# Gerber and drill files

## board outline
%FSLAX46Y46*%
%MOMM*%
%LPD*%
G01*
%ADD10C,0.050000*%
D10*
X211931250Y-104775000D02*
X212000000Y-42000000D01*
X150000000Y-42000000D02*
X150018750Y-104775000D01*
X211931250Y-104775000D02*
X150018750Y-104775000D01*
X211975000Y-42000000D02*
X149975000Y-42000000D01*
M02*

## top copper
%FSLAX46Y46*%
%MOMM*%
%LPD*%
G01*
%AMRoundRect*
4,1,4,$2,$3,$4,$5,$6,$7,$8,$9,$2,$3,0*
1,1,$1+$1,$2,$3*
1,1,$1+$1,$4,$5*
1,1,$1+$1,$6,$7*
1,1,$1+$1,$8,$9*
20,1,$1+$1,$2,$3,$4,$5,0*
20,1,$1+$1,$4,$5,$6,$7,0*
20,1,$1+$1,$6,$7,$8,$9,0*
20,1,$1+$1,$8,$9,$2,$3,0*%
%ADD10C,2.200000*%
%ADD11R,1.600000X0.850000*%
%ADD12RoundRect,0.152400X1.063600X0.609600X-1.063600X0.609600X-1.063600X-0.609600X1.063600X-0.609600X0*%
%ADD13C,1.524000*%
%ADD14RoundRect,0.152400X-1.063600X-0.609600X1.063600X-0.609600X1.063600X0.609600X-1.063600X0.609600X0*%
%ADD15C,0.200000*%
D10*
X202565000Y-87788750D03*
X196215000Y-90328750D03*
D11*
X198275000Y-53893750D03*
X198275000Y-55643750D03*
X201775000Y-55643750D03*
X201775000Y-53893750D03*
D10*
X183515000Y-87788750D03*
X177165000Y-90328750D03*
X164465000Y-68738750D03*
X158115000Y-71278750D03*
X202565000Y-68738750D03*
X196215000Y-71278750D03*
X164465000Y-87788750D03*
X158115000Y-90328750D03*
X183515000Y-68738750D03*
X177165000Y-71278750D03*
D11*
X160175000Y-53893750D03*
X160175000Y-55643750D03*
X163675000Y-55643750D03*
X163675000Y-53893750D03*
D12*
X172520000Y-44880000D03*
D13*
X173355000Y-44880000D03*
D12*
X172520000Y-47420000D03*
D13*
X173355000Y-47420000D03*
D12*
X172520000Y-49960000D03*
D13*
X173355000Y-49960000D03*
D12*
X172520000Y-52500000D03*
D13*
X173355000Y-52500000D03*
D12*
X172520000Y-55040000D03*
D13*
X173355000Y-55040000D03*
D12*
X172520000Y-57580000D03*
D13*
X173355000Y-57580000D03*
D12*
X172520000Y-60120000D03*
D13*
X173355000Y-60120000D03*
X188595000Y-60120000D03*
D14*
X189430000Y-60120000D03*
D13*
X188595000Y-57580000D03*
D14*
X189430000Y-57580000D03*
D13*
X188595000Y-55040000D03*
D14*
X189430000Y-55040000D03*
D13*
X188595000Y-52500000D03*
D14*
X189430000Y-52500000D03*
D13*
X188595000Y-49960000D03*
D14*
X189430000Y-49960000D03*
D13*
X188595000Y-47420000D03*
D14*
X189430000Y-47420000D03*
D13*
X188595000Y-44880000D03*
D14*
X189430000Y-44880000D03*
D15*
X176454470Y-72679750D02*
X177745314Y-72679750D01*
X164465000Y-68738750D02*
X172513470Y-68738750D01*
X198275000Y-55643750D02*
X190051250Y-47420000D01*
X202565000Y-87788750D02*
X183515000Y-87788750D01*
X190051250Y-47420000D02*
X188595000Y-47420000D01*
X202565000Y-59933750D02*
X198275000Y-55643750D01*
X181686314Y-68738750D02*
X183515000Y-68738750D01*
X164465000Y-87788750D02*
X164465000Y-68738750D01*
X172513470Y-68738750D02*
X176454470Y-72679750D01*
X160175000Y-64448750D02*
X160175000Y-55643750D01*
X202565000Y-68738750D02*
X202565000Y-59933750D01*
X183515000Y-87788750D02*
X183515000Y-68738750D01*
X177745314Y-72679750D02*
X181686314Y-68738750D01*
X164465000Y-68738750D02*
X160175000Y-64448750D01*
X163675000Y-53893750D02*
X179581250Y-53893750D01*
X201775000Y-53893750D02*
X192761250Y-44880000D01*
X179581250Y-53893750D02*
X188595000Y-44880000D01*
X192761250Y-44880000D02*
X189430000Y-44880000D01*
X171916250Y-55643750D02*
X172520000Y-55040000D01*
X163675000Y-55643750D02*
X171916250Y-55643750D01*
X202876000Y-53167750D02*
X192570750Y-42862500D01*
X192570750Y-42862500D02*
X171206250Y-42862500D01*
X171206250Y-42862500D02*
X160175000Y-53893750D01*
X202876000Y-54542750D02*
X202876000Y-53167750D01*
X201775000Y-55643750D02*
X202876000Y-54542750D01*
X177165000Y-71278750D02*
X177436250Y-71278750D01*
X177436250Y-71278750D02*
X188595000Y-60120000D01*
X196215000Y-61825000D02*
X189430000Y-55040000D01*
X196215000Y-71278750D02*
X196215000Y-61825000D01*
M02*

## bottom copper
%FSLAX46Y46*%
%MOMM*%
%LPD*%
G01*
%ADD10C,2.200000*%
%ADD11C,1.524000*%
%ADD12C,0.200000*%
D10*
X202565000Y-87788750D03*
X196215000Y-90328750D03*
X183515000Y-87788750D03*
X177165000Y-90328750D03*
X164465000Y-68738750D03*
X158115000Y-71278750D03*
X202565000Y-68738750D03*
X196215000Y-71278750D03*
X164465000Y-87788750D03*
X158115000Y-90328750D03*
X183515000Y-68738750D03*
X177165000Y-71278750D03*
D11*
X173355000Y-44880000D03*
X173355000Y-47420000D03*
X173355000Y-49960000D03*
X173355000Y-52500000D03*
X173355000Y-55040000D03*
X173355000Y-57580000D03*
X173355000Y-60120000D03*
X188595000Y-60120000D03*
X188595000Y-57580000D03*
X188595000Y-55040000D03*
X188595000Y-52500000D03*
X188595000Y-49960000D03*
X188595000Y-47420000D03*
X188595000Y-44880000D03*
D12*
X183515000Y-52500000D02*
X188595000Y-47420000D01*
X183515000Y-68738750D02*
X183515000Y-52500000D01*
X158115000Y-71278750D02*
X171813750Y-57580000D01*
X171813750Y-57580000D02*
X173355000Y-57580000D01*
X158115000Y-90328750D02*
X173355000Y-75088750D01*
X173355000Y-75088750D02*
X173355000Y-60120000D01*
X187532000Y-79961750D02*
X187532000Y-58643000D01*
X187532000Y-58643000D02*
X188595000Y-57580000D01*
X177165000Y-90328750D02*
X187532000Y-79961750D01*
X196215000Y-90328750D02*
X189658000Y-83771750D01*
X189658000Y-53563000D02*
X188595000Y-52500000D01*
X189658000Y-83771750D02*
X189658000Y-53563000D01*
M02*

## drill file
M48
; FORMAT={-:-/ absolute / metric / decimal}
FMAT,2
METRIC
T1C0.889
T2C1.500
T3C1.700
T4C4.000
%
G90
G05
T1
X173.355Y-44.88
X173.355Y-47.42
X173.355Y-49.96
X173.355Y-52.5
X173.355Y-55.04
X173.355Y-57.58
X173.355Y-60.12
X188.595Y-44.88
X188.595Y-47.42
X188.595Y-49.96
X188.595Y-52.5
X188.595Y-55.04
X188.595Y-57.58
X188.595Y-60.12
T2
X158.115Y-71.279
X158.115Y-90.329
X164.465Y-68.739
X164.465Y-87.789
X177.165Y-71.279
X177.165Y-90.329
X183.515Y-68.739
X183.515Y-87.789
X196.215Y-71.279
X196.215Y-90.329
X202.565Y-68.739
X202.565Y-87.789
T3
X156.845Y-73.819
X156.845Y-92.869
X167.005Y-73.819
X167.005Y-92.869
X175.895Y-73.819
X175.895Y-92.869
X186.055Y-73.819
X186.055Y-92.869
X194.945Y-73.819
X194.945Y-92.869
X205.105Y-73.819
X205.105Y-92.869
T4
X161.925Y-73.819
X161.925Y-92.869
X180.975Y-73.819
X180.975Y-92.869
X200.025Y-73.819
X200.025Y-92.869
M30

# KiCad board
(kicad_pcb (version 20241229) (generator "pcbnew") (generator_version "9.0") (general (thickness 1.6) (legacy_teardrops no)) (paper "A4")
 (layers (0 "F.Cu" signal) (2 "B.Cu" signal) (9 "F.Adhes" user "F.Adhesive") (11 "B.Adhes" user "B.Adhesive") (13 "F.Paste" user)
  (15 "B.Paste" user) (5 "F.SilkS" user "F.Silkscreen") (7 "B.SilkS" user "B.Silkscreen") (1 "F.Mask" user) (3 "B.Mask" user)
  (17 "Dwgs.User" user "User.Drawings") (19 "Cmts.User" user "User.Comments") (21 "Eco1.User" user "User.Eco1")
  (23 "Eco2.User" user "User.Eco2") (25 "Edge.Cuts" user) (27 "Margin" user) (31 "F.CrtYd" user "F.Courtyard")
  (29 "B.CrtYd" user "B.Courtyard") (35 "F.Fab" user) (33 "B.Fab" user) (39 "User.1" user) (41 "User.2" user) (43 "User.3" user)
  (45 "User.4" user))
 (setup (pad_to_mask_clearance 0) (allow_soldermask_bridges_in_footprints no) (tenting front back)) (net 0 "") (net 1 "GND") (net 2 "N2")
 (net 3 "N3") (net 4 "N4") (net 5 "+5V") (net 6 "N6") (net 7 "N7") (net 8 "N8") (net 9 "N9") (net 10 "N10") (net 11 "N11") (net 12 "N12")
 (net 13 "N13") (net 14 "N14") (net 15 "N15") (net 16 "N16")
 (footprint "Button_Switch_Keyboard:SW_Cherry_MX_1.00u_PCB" (layer "F.Cu") (at 202.565 87.78875)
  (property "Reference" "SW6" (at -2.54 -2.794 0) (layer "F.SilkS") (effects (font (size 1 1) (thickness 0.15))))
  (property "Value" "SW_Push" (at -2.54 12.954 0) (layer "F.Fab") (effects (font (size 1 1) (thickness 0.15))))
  (pad "" np_thru_hole circle (at -7.62 5.08) (size 1.7 1.7) (drill 1.7) (layers "*.Cu" "*.Mask"))
  (pad "" np_thru_hole circle (at -2.54 5.08) (size 4 4) (drill 4) (layers "*.Cu" "*.Mask"))
  (pad "" np_thru_hole circle (at 2.54 5.08) (size 1.7 1.7) (drill 1.7) (layers "*.Cu" "*.Mask"))
  (pad "1" thru_hole circle (at 0 0) (size 2.2 2.2) (drill 1.5) (layers "*.Cu" "*.Mask") (remove_unused_layers no) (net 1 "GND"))
  (pad "2" thru_hole circle (at -6.35 2.54) (size 2.2 2.2) (drill 1.5) (layers "*.Cu" "*.Mask") (remove_unused_layers no) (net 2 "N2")))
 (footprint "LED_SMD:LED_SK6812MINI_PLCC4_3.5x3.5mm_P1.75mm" (layer "F.Cu") (at 200.025 54.76875)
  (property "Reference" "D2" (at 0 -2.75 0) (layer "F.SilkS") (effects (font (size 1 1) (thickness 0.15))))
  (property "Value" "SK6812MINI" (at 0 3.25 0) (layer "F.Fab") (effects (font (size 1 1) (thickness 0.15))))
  (pad "1" smd rect (at -1.75 -0.875) (size 1.6 0.85) (layers "F.Cu" "F.Mask" "F.Paste") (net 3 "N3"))
  (pad "2" smd rect (at -1.75 0.875) (size 1.6 0.85) (layers "F.Cu" "F.Mask" "F.Paste") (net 1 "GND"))
  (pad "3" smd rect (at 1.75 0.875) (size 1.6 0.85) (layers "F.Cu" "F.Mask" "F.Paste") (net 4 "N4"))
  (pad "4" smd rect (at 1.75 -0.875) (size 1.6 0.85) (layers "F.Cu" "F.Mask" "F.Paste") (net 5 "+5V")))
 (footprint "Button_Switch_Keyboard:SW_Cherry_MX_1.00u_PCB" (layer "F.Cu") (at 183.515 87.78875)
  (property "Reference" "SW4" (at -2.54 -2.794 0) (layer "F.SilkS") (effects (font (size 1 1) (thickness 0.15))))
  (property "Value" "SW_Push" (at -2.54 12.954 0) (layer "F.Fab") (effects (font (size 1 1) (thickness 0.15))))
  (pad "" np_thru_hole circle (at -7.62 5.08) (size 1.7 1.7) (drill 1.7) (layers "*.Cu" "*.Mask"))
  (pad "" np_thru_hole circle (at -2.54 5.08) (size 4 4) (drill 4) (layers "*.Cu" "*.Mask"))
  (pad "" np_thru_hole circle (at 2.54 5.08) (size 1.7 1.7) (drill 1.7) (layers "*.Cu" "*.Mask"))
  (pad "1" thru_hole circle (at 0 0) (size 2.2 2.2) (drill 1.5) (layers "*.Cu" "*.Mask") (remove_unused_layers no) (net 1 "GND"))
  (pad "2" thru_hole circle (at -6.35 2.54) (size 2.2 2.2) (drill 1.5) (layers "*.Cu" "*.Mask") (remove_unused_layers no) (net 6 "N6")))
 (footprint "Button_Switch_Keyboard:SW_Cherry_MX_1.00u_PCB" (layer "F.Cu") (at 164.465 68.73875)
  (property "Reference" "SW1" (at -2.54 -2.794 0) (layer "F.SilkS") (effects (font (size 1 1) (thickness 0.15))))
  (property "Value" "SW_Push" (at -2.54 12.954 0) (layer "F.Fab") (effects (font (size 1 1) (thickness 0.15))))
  (pad "" np_thru_hole circle (at -7.62 5.08) (size 1.7 1.7) (drill 1.7) (layers "*.Cu" "*.Mask"))
  (pad "" np_thru_hole circle (at -2.54 5.08) (size 4 4) (drill 4) (layers "*.Cu" "*.Mask"))
  (pad "" np_thru_hole circle (at 2.54 5.08) (size 1.7 1.7) (drill 1.7) (layers "*.Cu" "*.Mask"))
  (pad "1" thru_hole circle (at 0 0) (size 2.2 2.2) (drill 1.5) (layers "*.Cu" "*.Mask") (remove_unused_layers no) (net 1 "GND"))
  (pad "2" thru_hole circle (at -6.35 2.54) (size 2.2 2.2) (drill 1.5) (layers "*.Cu" "*.Mask") (remove_unused_layers no) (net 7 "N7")))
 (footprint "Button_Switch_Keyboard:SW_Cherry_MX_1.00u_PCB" (layer "F.Cu") (at 202.565 68.73875)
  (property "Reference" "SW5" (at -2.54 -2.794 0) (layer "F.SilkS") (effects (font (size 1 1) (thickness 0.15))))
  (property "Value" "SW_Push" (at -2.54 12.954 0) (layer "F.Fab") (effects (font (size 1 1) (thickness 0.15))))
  (pad "" np_thru_hole circle (at -7.62 5.08) (size 1.7 1.7) (drill 1.7) (layers "*.Cu" "*.Mask"))
  (pad "" np_thru_hole circle (at -2.54 5.08) (size 4 4) (drill 4) (layers "*.Cu" "*.Mask"))
  (pad "" np_thru_hole circle (at 2.54 5.08) (size 1.7 1.7) (drill 1.7) (layers "*.Cu" "*.Mask"))
  (pad "1" thru_hole circle (at 0 0) (size 2.2 2.2) (drill 1.5) (layers "*.Cu" "*.Mask") (remove_unused_layers no) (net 1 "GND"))
  (pad "2" thru_hole circle (at -6.35 2.54) (size 2.2 2.2) (drill 1.5) (layers "*.Cu" "*.Mask") (remove_unused_layers no) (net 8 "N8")))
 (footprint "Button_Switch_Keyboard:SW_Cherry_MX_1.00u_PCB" (layer "F.Cu") (at 164.465 87.78875)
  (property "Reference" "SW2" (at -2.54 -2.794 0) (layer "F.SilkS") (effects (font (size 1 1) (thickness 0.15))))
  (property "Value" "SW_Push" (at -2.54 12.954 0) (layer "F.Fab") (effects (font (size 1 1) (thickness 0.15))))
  (pad "" np_thru_hole circle (at -7.62 5.08) (size 1.7 1.7) (drill 1.7) (layers "*.Cu" "*.Mask"))
  (pad "" np_thru_hole circle (at -2.54 5.08) (size 4 4) (drill 4) (layers "*.Cu" "*.Mask"))
  (pad "" np_thru_hole circle (at 2.54 5.08) (size 1.7 1.7) (drill 1.7) (layers "*.Cu" "*.Mask"))
  (pad "1" thru_hole circle (at 0 0) (size 2.2 2.2) (drill 1.5) (layers "*.Cu" "*.Mask") (remove_unused_layers no) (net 1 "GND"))
  (pad "2" thru_hole circle (at -6.35 2.54) (size 2.2 2.2) (drill 1.5) (layers "*.Cu" "*.Mask") (remove_unused_layers no) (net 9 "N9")))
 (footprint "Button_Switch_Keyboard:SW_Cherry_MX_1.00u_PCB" (layer "F.Cu") (at 183.515 68.73875)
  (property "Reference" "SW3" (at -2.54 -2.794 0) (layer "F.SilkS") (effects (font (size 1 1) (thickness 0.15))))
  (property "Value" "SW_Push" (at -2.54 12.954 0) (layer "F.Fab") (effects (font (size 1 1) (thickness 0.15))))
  (pad "" np_thru_hole circle (at -7.62 5.08) (size 1.7 1.7) (drill 1.7) (layers "*.Cu" "*.Mask"))
  (pad "" np_thru_hole circle (at -2.54 5.08) (size 4 4) (drill 4) (layers "*.Cu" "*.Mask"))
  (pad "" np_thru_hole circle (at 2.54 5.08) (size 1.7 1.7) (drill 1.7) (layers "*.Cu" "*.Mask"))
  (pad "1" thru_hole circle (at 0 0) (size 2.2 2.2) (drill 1.5) (layers "*.Cu" "*.Mask") (remove_unused_layers no) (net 1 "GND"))
  (pad "2" thru_hole circle (at -6.35 2.54) (size 2.2 2.2) (drill 1.5) (layers "*.Cu" "*.Mask") (remove_unused_layers no) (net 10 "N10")))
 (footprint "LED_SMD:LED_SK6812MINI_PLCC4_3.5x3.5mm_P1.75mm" (layer "F.Cu") (at 161.925 54.76875)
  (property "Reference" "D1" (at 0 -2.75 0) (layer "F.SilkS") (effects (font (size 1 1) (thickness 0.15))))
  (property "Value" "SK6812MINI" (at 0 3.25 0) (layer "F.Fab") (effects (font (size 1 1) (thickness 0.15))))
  (pad "1" smd rect (at -1.75 -0.875) (size 1.6 0.85) (layers "F.Cu" "F.Mask" "F.Paste") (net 4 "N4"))
  (pad "2" smd rect (at -1.75 0.875) (size 1.6 0.85) (layers "F.Cu" "F.Mask" "F.Paste") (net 1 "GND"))
  (pad "3" smd rect (at 1.75 0.875) (size 1.6 0.85) (layers "F.Cu" "F.Mask" "F.Paste") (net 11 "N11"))
  (pad "4" smd rect (at 1.75 -0.875) (size 1.6 0.85) (layers "F.Cu" "F.Mask" "F.Paste") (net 5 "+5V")))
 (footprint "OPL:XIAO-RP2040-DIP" (layer "F.Cu") (at 180.975 52.5)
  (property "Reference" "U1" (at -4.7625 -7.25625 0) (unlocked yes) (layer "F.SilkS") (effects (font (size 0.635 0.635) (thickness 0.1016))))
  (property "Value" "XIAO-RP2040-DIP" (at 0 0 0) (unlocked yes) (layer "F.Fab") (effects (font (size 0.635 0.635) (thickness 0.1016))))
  (pad "1" smd roundrect (at -8.455 -7.62 180) (size 2.432 1.524) (layers "F.Cu" "F.Mask") (roundrect_rratio 0.1) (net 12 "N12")
   (thermal_bridge_angle 45))
  (pad "1" thru_hole circle (at -7.62 -7.62 180) (size 1.524 1.524) (drill 0.889) (layers "*.Cu" "*.Mask") (remove_unused_layers no)
   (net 12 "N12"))
  (pad "2" smd roundrect (at -8.455 -5.08 180) (size 2.432 1.524) (layers "F.Cu" "F.Mask") (roundrect_rratio 0.1) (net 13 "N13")
   (thermal_bridge_angle 45))
  (pad "2" thru_hole circle (at -7.62 -5.08 180) (size 1.524 1.524) (drill 0.889) (layers "*.Cu" "*.Mask") (remove_unused_layers no)
   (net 13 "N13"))
  (pad "3" smd roundrect (at -8.455 -2.54 180) (size 2.432 1.524) (layers "F.Cu" "F.Mask") (roundrect_rratio 0.1) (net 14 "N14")
   (thermal_bridge_angle 45))
  (pad "3" thru_hole circle (at -7.62 -2.54 180) (size 1.524 1.524) (drill 0.889) (layers "*.Cu" "*.Mask") (remove_unused_layers no)
   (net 14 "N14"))
  (pad "4" smd roundrect (at -8.455 0 180) (size 2.432 1.524) (layers "F.Cu" "F.Mask") (roundrect_rratio 0.1) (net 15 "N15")
   (thermal_bridge_angle 45))
  (pad "4" thru_hole circle (at -7.62 0 180) (size 1.524 1.524) (drill 0.889) (layers "*.Cu" "*.Mask") (remove_unused_layers no)
   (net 15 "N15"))
  (pad "5" smd roundrect (at -8.455 2.54 180) (size 2.432 1.524) (layers "F.Cu" "F.Mask") (roundrect_rratio 0.1) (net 11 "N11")
   (thermal_bridge_angle 45))
  (pad "5" thru_hole circle (at -7.62 2.54 180) (size 1.524 1.524) (drill 0.889) (layers "*.Cu" "*.Mask") (remove_unused_layers no)
   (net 11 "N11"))
  (pad "6" smd roundrect (at -8.455 5.08 180) (size 2.432 1.524) (layers "F.Cu" "F.Mask") (roundrect_rratio 0.1) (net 7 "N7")
   (thermal_bridge_angle 45))
  (pad "6" thru_hole circle (at -7.62 5.08 180) (size 1.524 1.524) (drill 0.889) (layers "*.Cu" "*.Mask") (remove_unused_layers no)
   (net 7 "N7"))
  (pad "7" smd roundrect (at -8.455 7.62 180) (size 2.432 1.524) (layers "F.Cu" "F.Mask") (roundrect_rratio 0.1) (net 9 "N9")
   (thermal_bridge_angle 45))
  (pad "7" thru_hole circle (at -7.62 7.62 180) (size 1.524 1.524) (drill 0.889) (layers "*.Cu" "*.Mask") (remove_unused_layers no)
   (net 9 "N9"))
  (pad "8" thru_hole circle (at 7.62 7.62) (size 1.524 1.524) (drill 0.889) (layers "*.Cu" "*.Mask") (remove_unused_layers no)
   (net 10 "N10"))
  (pad "8" smd roundrect (at 8.455 7.62) (size 2.432 1.524) (layers "F.Cu" "F.Mask") (roundrect_rratio 0.1) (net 10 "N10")
   (thermal_bridge_angle 45))
  (pad "9" thru_hole circle (at 7.62 5.08) (size 1.524 1.524) (drill 0.889) (layers "*.Cu" "*.Mask") (remove_unused_layers no) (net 6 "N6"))
  (pad "9" smd roundrect (at 8.455 5.08) (size 2.432 1.524) (layers "F.Cu" "F.Mask") (roundrect_rratio 0.1) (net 6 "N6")
   (thermal_bridge_angle 45))
  (pad "10" thru_hole circle (at 7.62 2.54) (size 1.524 1.524) (drill 0.889) (layers "*.Cu" "*.Mask") (remove_unused_layers no) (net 8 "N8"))
  (pad "10" smd roundrect (at 8.455 2.54) (size 2.432 1.524) (layers "F.Cu" "F.Mask") (roundrect_rratio 0.1) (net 8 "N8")
   (thermal_bridge_angle 45))
  (pad "11" thru_hole circle (at 7.62 0) (size 1.524 1.524) (drill 0.889) (layers "*.Cu" "*.Mask") (remove_unused_layers no) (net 2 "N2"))
  (pad "11" smd roundrect (at 8.455 0) (size 2.432 1.524) (layers "F.Cu" "F.Mask") (roundrect_rratio 0.1) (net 2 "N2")
   (thermal_bridge_angle 45))
  (pad "12" thru_hole circle (at 7.62 -2.54) (size 1.524 1.524) (drill 0.889) (layers "*.Cu" "*.Mask") (remove_unused_layers no)
   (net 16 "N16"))
  (pad "12" smd roundrect (at 8.455 -2.54) (size 2.432 1.524) (layers "F.Cu" "F.Mask") (roundrect_rratio 0.1) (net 16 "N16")
   (thermal_bridge_angle 45))
  (pad "13" thru_hole circle (at 7.62 -5.08) (size 1.524 1.524) (drill 0.889) (layers "*.Cu" "*.Mask") (remove_unused_layers no)
   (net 1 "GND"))
  (pad "13" smd roundrect (at 8.455 -5.08) (size 2.432 1.524) (layers "F.Cu" "F.Mask") (roundrect_rratio 0.1) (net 1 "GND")
   (thermal_bridge_angle 45))
  (pad "14" thru_hole circle (at 7.62 -7.62) (size 1.524 1.524) (drill 0.889) (layers "*.Cu" "*.Mask") (remove_unused_layers no)
   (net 5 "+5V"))
  (pad "14" smd roundrect (at 8.455 -7.62) (size 2.432 1.524) (layers "F.Cu" "F.Mask") (roundrect_rratio 0.1) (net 5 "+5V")
   (thermal_bridge_angle 45)))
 (gr_line (start 211.93125 104.775) (end 212 42) (stroke (width 0.05) (type default)) (layer "Edge.Cuts"))
 (gr_line (start 150 42) (end 150.01875 104.775) (stroke (width 0.05) (type default)) (layer "Edge.Cuts"))
 (gr_line (start 211.93125 104.775) (end 150.01875 104.775) (stroke (width 0.05) (type default)) (layer "Edge.Cuts"))
 (gr_line (start 211.975 42) (end 149.975 42) (stroke (width 0.05) (type default)) (layer "Edge.Cuts"))
 (segment (start 176.45447 72.67975) (end 177.745314 72.67975) (width 0.2) (layer "F.Cu") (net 1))
 (segment (start 164.465 68.73875) (end 172.51347 68.73875) (width 0.2) (layer "F.Cu") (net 1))
 (segment (start 198.275 55.64375) (end 190.05125 47.42) (width 0.2) (layer "F.Cu") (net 1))
 (segment (start 202.565 87.78875) (end 183.515 87.78875) (width 0.2) (layer "F.Cu") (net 1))
 (segment (start 190.05125 47.42) (end 188.595 47.42) (width 0.2) (layer "F.Cu") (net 1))
 (segment (start 202.565 59.93375) (end 198.275 55.64375) (width 0.2) (layer "F.Cu") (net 1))
 (segment (start 181.686314 68.73875) (end 183.515 68.73875) (width 0.2) (layer "F.Cu") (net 1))
 (segment (start 164.465 87.78875) (end 164.465 68.73875) (width 0.2) (layer "F.Cu") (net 1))
 (segment (start 172.51347 68.73875) (end 176.45447 72.67975) (width 0.2) (layer "F.Cu") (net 1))
 (segment (start 160.175 64.44875) (end 160.175 55.64375) (width 0.2) (layer "F.Cu") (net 1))
 (segment (start 202.565 68.73875) (end 202.565 59.93375) (width 0.2) (layer "F.Cu") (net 1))
 (segment (start 183.515 87.78875) (end 183.515 68.73875) (width 0.2) (layer "F.Cu") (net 1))
 (segment (start 177.745314 72.67975) (end 181.686314 68.73875) (width 0.2) (layer "F.Cu") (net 1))
 (segment (start 164.465 68.73875) (end 160.175 64.44875) (width 0.2) (layer "F.Cu") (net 1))
 (segment (start 183.515 52.5) (end 188.595 47.42) (width 0.2) (layer "B.Cu") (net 1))
 (segment (start 183.515 68.73875) (end 183.515 52.5) (width 0.2) (layer "B.Cu") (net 1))
 (segment (start 163.675 53.89375) (end 179.58125 53.89375) (width 0.2) (layer "F.Cu") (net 5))
 (segment (start 201.775 53.89375) (end 192.76125 44.88) (width 0.2) (layer "F.Cu") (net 5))
 (segment (start 179.58125 53.89375) (end 188.595 44.88) (width 0.2) (layer "F.Cu") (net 5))
 (segment (start 192.76125 44.88) (end 189.43 44.88) (width 0.2) (layer "F.Cu") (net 5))
 (segment (start 171.91625 55.64375) (end 172.52 55.04) (width 0.2) (layer "F.Cu") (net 11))
 (segment (start 163.675 55.64375) (end 171.91625 55.64375) (width 0.2) (layer "F.Cu") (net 11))
 (segment (start 202.876 53.16775) (end 192.57075 42.8625) (width 0.2) (layer "F.Cu") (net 4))
 (segment (start 192.57075 42.8625) (end 171.20625 42.8625) (width 0.2) (layer "F.Cu") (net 4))
 (segment (start 171.20625 42.8625) (end 160.175 53.89375) (width 0.2) (layer "F.Cu") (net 4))
 (segment (start 202.876 54.54275) (end 202.876 53.16775) (width 0.2) (layer "F.Cu") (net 4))
 (segment (start 201.775 55.64375) (end 202.876 54.54275) (width 0.2) (layer "F.Cu") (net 4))
 (segment (start 158.115 71.27875) (end 171.81375 57.58) (width 0.2) (layer "B.Cu") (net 7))
 (segment (start 171.81375 57.58) (end 173.355 57.58) (width 0.2) (layer "B.Cu") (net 7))
 (segment (start 158.115 90.32875) (end 173.355 75.08875) (width 0.2) (layer "B.Cu") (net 9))
 (segment (start 173.355 75.08875) (end 173.355 60.12) (width 0.2) (layer "B.Cu") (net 9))
 (segment (start 177.165 71.27875) (end 177.43625 71.27875) (width 0.2) (layer "F.Cu") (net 10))
 (segment (start 177.43625 71.27875) (end 188.595 60.12) (width 0.2) (layer "F.Cu") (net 10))
 (segment (start 187.532 79.96175) (end 187.532 58.643) (width 0.2) (layer "B.Cu") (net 6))
 (segment (start 187.532 58.643) (end 188.595 57.58) (width 0.2) (layer "B.Cu") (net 6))
 (segment (start 177.165 90.32875) (end 187.532 79.96175) (width 0.2) (layer "B.Cu") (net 6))
 (segment (start 196.215 61.825) (end 189.43 55.04) (width 0.2) (layer "F.Cu") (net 8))
 (segment (start 196.215 71.27875) (end 196.215 61.825) (width 0.2) (layer "F.Cu") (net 8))
 (segment (start 196.215 90.32875) (end 189.658 83.77175) (width 0.2) (layer "B.Cu") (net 2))
 (segment (start 189.658 53.563) (end 188.595 52.5) (width 0.2) (layer "B.Cu") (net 2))
 (segment (start 189.658 83.77175) (end 189.658 53.563) (width 0.2) (layer "B.Cu") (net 2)))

